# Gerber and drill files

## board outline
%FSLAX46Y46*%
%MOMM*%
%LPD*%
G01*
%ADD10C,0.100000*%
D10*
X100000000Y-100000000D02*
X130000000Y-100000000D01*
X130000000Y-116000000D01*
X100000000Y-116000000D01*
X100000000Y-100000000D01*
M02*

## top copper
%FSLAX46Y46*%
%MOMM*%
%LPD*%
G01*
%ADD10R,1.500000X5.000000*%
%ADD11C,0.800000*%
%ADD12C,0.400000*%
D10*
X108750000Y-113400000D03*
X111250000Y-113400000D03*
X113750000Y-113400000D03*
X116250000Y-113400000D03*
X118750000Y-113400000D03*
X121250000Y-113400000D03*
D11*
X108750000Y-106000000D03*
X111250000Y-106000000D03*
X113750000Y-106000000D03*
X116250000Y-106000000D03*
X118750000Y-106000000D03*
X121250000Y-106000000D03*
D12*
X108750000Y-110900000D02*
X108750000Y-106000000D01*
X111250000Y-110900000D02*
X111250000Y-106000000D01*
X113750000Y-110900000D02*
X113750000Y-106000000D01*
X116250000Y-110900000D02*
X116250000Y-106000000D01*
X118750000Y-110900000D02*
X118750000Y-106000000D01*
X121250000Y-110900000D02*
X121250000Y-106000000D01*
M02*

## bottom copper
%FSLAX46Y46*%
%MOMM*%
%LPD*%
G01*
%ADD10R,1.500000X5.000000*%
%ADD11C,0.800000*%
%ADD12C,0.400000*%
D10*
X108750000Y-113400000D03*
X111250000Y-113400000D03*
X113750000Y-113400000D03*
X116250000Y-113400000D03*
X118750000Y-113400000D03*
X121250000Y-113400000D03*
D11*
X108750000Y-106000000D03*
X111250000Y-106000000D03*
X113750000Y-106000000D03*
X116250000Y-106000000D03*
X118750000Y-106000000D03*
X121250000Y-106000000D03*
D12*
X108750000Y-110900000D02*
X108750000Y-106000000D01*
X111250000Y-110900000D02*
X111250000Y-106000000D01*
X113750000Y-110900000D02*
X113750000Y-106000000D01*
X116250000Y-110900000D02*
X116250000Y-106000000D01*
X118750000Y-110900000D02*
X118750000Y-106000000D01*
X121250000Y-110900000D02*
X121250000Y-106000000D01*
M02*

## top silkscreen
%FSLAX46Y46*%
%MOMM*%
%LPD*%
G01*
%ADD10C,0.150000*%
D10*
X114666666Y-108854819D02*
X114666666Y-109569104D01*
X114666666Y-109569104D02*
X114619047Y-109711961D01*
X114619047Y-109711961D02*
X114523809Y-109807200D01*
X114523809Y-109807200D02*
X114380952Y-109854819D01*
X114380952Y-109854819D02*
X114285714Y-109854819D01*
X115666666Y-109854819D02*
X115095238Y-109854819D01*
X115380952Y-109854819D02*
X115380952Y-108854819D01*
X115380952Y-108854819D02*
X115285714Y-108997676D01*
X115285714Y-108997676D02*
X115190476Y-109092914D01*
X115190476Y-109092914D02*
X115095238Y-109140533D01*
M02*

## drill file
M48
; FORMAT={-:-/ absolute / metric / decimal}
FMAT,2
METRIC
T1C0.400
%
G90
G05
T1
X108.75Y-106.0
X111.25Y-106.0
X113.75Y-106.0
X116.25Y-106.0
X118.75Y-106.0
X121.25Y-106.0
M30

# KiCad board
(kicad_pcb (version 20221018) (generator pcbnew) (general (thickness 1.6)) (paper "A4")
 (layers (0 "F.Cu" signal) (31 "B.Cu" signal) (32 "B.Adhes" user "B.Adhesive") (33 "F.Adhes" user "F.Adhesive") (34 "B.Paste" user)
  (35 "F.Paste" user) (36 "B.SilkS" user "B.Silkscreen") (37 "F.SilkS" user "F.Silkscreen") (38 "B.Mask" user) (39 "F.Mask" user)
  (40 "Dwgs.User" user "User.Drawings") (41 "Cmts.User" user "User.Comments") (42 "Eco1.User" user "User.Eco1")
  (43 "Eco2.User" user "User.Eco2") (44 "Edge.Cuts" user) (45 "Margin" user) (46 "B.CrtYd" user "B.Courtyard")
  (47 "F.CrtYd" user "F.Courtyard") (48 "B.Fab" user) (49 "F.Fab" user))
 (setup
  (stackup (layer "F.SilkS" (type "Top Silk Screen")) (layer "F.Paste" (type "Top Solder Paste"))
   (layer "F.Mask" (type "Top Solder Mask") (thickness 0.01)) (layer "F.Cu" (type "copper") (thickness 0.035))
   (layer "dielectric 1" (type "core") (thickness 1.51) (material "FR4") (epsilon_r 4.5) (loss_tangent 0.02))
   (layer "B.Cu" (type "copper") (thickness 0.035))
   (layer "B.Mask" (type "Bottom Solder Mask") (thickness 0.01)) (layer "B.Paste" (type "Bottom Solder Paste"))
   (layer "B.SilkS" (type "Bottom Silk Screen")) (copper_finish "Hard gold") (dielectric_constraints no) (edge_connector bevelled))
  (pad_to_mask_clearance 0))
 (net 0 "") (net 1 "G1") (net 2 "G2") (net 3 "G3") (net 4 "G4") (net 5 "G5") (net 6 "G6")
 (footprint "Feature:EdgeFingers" (layer "F.Cu") (at 115 113.4)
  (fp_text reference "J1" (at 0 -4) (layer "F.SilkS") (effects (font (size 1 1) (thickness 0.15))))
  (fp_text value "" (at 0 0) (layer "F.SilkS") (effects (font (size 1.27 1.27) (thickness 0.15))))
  (pad "A1" connect rect (at -6.25 0) (size 1.5 5) (layers "F.Cu" "F.Mask") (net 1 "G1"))
  (pad "A2" connect rect (at -3.75 0) (size 1.5 5) (layers "F.Cu" "F.Mask") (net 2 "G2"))
  (pad "A3" connect rect (at -1.25 0) (size 1.5 5) (layers "F.Cu" "F.Mask") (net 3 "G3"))
  (pad "A4" connect rect (at 1.25 0) (size 1.5 5) (layers "F.Cu" "F.Mask") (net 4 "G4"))
  (pad "A5" connect rect (at 3.75 0) (size 1.5 5) (layers "F.Cu" "F.Mask") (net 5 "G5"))
  (pad "A6" connect rect (at 6.25 0) (size 1.5 5) (layers "F.Cu" "F.Mask") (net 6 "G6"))
  (pad "B1" connect rect (at -6.25 0) (size 1.5 5) (layers "B.Cu" "B.Mask") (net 1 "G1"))
  (pad "B2" connect rect (at -3.75 0) (size 1.5 5) (layers "B.Cu" "B.Mask") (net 2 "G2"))
  (pad "B3" connect rect (at -1.25 0) (size 1.5 5) (layers "B.Cu" "B.Mask") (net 3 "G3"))
  (pad "B4" connect rect (at 1.25 0) (size 1.5 5) (layers "B.Cu" "B.Mask") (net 4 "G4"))
  (pad "B5" connect rect (at 3.75 0) (size 1.5 5) (layers "B.Cu" "B.Mask") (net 5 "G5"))
  (pad "B6" connect rect (at 6.25 0) (size 1.5 5) (layers "B.Cu" "B.Mask") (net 6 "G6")))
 (gr_rect (start 100 100) (end 130 116) (stroke (width 0.1) (type solid)) (fill none) (layer "Edge.Cuts"))
 (segment (start 108.75 110.9) (end 108.75 106) (width 0.4) (layer "F.Cu") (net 1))
 (via (at 108.75 106) (size 0.8) (drill 0.4) (layers "F.Cu" "B.Cu") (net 1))
 (segment (start 108.75 110.9) (end 108.75 106) (width 0.4) (layer "B.Cu") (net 1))
 (segment (start 111.25 110.9) (end 111.25 106) (width 0.4) (layer "F.Cu") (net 2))
 (via (at 111.25 106) (size 0.8) (drill 0.4) (layers "F.Cu" "B.Cu") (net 2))
 (segment (start 111.25 110.9) (end 111.25 106) (width 0.4) (layer "B.Cu") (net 2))
 (segment (start 113.75 110.9) (end 113.75 106) (width 0.4) (layer "F.Cu") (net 3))
 (via (at 113.75 106) (size 0.8) (drill 0.4) (layers "F.Cu" "B.Cu") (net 3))
 (segment (start 113.75 110.9) (end 113.75 106) (width 0.4) (layer "B.Cu") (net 3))
 (segment (start 116.25 110.9) (end 116.25 106) (width 0.4) (layer "F.Cu") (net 4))
 (via (at 116.25 106) (size 0.8) (drill 0.4) (layers "F.Cu" "B.Cu") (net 4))
 (segment (start 116.25 110.9) (end 116.25 106) (width 0.4) (layer "B.Cu") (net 4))
 (segment (start 118.75 110.9) (end 118.75 106) (width 0.4) (layer "F.Cu") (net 5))
 (via (at 118.75 106) (size 0.8) (drill 0.4) (layers "F.Cu" "B.Cu") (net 5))
 (segment (start 118.75 110.9) (end 118.75 106) (width 0.4) (layer "B.Cu") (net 5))
 (segment (start 121.25 110.9) (end 121.25 106) (width 0.4) (layer "F.Cu") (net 6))
 (via (at 121.25 106) (size 0.8) (drill 0.4) (layers "F.Cu" "B.Cu") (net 6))
 (segment (start 121.25 110.9) (end 121.25 106) (width 0.4) (layer "B.Cu") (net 6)))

